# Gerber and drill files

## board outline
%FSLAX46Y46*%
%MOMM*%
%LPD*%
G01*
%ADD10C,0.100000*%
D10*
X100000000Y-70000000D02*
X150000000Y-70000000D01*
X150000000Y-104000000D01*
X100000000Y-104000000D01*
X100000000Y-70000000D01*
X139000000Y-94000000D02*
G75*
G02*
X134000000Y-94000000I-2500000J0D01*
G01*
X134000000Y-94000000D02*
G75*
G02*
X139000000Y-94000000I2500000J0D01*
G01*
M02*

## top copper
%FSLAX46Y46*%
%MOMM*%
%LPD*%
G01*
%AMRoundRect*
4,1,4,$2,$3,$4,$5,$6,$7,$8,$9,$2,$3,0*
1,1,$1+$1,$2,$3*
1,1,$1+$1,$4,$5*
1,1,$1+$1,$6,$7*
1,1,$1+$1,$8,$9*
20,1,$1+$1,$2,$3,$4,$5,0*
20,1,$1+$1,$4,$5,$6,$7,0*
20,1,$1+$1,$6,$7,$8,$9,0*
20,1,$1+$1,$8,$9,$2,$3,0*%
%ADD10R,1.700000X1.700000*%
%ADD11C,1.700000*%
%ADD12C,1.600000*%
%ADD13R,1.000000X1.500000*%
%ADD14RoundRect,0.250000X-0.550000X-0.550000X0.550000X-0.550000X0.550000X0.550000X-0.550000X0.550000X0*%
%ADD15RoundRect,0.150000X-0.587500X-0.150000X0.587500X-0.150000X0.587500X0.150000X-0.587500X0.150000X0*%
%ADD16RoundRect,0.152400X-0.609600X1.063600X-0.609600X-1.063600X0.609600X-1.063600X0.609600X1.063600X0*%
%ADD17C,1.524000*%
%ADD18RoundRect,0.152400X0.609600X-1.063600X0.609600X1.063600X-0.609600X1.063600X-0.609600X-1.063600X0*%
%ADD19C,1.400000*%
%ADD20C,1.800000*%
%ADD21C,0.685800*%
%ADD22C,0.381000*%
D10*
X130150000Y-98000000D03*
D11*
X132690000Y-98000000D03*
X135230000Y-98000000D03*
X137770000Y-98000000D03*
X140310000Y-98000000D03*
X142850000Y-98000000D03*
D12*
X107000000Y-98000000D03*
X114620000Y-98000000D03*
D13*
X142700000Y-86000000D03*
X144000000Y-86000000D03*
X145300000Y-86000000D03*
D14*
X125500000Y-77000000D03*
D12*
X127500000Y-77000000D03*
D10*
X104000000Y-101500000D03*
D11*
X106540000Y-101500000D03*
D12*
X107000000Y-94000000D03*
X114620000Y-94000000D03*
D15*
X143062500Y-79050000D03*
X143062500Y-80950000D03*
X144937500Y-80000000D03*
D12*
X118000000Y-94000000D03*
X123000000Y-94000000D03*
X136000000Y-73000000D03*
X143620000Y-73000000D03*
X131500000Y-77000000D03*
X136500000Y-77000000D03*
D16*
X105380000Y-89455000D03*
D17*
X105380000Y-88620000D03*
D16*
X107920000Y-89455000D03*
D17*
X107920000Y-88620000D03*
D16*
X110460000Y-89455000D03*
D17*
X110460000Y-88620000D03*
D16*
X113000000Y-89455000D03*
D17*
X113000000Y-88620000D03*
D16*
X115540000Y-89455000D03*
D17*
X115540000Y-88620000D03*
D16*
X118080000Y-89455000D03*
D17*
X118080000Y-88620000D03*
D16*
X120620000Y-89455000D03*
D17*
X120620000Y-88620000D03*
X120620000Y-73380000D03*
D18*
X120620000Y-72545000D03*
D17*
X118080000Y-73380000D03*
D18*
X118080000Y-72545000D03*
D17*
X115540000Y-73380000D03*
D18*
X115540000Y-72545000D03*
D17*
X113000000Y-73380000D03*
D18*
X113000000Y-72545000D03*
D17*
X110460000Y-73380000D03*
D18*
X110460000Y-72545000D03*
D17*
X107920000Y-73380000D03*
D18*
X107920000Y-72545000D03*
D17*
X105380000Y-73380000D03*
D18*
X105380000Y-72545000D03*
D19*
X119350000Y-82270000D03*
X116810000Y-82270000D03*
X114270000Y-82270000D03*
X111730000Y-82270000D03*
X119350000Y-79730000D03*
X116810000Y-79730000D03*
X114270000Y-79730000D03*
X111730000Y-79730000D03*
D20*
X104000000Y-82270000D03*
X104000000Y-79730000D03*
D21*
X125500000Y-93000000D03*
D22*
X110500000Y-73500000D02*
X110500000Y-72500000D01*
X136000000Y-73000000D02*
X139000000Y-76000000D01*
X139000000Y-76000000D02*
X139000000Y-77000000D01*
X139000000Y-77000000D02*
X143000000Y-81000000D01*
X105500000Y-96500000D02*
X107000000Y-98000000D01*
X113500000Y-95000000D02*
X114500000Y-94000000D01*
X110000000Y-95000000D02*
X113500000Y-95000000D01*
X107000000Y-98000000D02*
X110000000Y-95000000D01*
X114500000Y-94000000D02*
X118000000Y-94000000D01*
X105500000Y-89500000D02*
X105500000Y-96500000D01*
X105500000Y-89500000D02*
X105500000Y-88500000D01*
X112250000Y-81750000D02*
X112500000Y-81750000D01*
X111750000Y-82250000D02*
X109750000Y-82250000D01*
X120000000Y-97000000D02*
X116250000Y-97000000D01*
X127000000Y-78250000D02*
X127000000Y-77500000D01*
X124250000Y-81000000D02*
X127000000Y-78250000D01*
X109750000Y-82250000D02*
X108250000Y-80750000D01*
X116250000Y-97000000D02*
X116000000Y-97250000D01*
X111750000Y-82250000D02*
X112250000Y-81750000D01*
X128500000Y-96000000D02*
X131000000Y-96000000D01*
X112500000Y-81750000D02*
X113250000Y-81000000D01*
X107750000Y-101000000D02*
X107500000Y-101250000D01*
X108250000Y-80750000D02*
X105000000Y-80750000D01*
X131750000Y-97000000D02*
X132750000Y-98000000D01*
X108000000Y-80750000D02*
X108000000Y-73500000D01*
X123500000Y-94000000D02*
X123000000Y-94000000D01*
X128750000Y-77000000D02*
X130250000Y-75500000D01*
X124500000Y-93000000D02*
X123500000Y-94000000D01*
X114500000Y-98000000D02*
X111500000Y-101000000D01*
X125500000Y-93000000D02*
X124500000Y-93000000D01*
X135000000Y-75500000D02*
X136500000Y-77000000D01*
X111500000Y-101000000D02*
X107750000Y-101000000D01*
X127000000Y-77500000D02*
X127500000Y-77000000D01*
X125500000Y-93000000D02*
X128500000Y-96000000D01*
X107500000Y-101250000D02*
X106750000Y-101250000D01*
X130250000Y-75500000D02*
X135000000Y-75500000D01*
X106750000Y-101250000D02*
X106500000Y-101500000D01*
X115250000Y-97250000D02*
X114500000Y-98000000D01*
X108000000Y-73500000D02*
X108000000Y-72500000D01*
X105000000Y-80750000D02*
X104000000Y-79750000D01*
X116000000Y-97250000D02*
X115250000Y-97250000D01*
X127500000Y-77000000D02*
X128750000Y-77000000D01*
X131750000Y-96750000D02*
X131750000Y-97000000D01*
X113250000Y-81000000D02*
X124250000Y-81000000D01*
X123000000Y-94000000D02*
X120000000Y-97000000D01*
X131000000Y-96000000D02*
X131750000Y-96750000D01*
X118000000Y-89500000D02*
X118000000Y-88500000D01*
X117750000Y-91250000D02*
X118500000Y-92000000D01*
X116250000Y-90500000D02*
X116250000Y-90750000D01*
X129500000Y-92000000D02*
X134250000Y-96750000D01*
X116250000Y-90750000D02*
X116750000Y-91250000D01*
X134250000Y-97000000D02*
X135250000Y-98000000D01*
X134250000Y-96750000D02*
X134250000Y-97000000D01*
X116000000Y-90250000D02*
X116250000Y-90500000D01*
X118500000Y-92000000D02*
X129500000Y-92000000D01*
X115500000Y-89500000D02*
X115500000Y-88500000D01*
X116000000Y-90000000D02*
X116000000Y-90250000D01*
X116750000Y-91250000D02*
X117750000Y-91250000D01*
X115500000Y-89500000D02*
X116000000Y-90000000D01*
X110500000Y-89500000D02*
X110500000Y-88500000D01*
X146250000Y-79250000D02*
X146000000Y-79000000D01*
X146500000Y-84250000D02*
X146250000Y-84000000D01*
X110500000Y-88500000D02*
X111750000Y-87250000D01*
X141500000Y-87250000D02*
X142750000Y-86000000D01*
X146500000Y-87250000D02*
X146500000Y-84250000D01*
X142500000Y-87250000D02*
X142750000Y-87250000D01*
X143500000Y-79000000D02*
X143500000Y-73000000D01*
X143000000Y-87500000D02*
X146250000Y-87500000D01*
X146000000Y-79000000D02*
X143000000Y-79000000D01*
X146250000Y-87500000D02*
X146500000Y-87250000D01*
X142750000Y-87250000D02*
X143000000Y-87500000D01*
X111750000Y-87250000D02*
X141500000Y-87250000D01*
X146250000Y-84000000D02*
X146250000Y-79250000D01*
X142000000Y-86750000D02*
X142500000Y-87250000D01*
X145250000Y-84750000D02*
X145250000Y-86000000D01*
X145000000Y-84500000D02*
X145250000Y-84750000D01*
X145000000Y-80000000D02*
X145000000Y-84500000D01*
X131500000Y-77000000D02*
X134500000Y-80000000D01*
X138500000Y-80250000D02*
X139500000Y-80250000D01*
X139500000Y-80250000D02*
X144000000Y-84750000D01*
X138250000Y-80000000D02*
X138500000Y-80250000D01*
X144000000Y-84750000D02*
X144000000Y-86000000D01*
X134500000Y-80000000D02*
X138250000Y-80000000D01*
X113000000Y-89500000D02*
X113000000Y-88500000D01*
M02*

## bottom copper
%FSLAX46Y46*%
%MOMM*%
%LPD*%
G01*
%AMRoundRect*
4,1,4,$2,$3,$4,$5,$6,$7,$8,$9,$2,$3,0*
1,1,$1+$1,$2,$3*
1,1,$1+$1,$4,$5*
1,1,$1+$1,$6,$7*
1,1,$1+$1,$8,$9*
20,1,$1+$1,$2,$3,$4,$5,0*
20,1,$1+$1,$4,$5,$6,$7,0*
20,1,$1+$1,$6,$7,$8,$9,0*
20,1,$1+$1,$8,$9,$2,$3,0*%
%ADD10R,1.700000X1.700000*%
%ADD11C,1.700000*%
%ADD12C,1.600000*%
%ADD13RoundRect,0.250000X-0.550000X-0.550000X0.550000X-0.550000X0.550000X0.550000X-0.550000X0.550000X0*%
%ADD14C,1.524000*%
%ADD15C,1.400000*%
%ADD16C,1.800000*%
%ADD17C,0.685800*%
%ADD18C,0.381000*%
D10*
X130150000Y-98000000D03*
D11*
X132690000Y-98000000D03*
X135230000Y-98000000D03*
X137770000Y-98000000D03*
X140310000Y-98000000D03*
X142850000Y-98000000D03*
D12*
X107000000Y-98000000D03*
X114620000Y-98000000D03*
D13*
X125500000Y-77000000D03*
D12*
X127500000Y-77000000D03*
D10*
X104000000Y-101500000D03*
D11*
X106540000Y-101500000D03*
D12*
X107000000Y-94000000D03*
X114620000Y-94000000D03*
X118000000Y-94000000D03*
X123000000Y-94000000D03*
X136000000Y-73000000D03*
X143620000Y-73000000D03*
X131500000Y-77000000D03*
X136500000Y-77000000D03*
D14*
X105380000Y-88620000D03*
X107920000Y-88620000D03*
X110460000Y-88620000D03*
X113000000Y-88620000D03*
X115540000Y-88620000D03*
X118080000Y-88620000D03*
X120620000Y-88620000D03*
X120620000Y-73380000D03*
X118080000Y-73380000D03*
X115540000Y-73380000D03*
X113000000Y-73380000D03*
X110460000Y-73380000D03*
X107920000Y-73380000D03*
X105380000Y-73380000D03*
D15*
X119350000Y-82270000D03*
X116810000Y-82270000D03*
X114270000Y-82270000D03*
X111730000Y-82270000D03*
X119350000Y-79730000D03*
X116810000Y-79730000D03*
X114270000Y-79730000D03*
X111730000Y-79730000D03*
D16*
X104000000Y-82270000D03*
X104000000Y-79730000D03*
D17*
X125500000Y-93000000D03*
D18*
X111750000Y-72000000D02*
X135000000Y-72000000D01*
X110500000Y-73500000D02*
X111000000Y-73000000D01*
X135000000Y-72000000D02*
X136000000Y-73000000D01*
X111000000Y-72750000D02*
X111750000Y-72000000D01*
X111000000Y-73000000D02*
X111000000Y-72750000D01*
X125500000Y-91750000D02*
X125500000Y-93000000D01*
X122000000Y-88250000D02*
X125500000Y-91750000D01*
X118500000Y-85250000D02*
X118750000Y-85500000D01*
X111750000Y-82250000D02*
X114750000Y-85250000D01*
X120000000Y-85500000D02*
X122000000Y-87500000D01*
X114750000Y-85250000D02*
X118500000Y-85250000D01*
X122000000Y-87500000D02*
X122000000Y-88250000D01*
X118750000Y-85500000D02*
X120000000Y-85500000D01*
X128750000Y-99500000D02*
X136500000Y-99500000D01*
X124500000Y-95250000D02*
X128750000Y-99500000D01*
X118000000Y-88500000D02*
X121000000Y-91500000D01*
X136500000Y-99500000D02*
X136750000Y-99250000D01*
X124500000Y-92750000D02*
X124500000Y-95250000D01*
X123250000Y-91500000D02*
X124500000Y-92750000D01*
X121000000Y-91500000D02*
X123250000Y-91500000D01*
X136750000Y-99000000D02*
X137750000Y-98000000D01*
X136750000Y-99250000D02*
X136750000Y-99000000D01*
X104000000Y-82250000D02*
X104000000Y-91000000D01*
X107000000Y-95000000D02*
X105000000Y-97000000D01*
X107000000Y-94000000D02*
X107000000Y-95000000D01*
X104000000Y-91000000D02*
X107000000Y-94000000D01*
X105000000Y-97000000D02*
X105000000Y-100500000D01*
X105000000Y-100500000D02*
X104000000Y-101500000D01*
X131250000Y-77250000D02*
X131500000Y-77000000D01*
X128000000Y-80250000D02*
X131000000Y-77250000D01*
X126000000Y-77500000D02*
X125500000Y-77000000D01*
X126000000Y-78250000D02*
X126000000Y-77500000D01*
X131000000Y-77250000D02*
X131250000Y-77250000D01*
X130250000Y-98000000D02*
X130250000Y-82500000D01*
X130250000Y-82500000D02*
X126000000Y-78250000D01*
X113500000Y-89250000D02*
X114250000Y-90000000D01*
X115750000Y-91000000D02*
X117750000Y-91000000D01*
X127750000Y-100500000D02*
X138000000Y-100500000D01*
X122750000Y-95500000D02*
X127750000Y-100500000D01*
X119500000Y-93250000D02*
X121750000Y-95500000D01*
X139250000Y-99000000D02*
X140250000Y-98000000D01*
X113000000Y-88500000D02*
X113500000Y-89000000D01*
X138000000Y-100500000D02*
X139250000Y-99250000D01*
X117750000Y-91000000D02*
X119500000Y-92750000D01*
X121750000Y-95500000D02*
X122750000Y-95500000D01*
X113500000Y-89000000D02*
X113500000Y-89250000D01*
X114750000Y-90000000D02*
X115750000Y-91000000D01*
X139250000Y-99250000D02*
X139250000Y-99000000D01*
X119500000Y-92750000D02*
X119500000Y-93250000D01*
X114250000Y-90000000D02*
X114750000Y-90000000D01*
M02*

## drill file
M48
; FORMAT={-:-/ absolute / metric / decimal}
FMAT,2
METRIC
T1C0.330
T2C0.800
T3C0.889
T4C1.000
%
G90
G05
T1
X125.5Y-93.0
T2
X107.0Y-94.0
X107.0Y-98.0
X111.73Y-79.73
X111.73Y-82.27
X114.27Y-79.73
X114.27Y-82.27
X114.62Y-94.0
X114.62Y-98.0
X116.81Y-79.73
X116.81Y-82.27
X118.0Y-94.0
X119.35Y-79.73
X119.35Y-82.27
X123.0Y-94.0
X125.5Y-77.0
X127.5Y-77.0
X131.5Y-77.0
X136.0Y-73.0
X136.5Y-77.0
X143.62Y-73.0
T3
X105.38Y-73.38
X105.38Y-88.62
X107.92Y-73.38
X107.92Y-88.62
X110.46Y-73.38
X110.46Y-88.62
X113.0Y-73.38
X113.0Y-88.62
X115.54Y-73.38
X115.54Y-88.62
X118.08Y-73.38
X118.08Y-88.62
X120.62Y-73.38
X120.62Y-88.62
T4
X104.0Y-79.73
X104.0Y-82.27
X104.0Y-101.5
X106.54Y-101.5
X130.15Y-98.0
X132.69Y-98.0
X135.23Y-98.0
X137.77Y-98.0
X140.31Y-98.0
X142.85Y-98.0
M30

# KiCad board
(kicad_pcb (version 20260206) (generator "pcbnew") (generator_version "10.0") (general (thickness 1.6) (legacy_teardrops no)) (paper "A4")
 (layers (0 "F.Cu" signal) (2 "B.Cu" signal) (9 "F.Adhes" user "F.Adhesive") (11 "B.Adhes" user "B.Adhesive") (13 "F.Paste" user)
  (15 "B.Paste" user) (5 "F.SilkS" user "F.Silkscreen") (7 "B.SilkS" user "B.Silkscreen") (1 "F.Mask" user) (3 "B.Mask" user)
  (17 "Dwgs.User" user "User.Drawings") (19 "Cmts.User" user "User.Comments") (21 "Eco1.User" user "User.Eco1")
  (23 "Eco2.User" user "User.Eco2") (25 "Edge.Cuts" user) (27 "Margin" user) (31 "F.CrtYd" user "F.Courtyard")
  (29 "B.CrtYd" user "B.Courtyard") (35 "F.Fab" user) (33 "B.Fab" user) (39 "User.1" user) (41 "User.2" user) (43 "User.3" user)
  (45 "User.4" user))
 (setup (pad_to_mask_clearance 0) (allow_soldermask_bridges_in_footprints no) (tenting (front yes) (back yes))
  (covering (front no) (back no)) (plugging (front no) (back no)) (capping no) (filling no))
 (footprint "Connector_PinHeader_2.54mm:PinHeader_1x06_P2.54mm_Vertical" (layer "F.Cu") (at 130.15 98 90)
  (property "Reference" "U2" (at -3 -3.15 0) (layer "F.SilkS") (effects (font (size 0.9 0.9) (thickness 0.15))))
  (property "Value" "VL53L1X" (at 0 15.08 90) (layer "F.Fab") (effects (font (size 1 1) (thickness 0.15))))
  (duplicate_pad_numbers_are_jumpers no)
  (pad "1" thru_hole rect (at 0 0 90) (size 1.7 1.7) (drill 1) (layers "*.Cu" "*.Mask") (remove_unused_layers no) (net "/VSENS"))
  (pad "2" thru_hole circle (at 0 2.54 90) (size 1.7 1.7) (drill 1) (layers "*.Cu" "*.Mask") (remove_unused_layers no) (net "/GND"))
  (pad "3" thru_hole circle (at 0 5.08 90) (size 1.7 1.7) (drill 1) (layers "*.Cu" "*.Mask") (remove_unused_layers no) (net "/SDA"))
  (pad "4" thru_hole circle (at 0 7.62 90) (size 1.7 1.7) (drill 1) (layers "*.Cu" "*.Mask") (remove_unused_layers no) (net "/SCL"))
  (pad "5" thru_hole circle (at 0 10.16 90) (size 1.7 1.7) (drill 1) (layers "*.Cu" "*.Mask") (remove_unused_layers no) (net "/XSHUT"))
  (pad "6" thru_hole circle (at 0 12.7 90) (size 1.7 1.7) (drill 1) (layers "*.Cu" "*.Mask") (remove_unused_layers no)
   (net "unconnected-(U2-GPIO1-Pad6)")))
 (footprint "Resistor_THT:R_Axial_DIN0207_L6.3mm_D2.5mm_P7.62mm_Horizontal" (layer "F.Cu") (at 107 98)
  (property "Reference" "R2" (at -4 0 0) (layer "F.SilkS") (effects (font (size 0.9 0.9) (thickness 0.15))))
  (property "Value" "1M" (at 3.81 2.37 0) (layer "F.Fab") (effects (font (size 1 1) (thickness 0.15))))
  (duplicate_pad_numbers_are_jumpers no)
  (pad "1" thru_hole circle (at 0 0) (size 1.6 1.6) (drill 0.8) (layers "*.Cu" "*.Mask") (remove_unused_layers no) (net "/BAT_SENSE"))
  (pad "2" thru_hole circle (at 7.62 0) (size 1.6 1.6) (drill 0.8) (layers "*.Cu" "*.Mask") (remove_unused_layers no) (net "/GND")))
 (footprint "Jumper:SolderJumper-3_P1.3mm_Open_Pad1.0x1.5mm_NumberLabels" (layer "F.Cu") (at 144 86)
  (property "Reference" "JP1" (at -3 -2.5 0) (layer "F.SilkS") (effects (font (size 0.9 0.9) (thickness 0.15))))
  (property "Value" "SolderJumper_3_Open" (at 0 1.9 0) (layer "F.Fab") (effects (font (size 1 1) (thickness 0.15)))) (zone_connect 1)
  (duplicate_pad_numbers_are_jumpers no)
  (pad "1" smd rect (at -1.3 0) (size 1 1.5) (layers "F.Cu" "F.Mask") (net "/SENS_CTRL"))
  (pad "2" smd rect (at 0 0) (size 1 1.5) (layers "F.Cu" "F.Mask") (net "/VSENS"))
  (pad "3" smd rect (at 1.3 0) (size 1 1.5) (layers "F.Cu" "F.Mask") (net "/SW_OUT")))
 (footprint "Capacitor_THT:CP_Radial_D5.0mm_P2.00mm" (layer "F.Cu") (at 125.5 77)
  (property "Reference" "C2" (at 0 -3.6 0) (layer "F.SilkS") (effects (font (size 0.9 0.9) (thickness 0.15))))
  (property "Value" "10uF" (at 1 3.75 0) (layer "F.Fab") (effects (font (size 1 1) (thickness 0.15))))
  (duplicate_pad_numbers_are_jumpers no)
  (pad "1" thru_hole roundrect (at 0 0) (size 1.6 1.6) (drill 0.8) (layers "*.Cu" "*.Mask") (remove_unused_layers no)
   (roundrect_rratio 0.15625) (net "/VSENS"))
  (pad "2" thru_hole circle (at 2 0) (size 1.6 1.6) (drill 0.8) (layers "*.Cu" "*.Mask") (remove_unused_layers no) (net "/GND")))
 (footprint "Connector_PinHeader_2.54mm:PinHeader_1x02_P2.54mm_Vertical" (layer "F.Cu") (at 104 101.5 90)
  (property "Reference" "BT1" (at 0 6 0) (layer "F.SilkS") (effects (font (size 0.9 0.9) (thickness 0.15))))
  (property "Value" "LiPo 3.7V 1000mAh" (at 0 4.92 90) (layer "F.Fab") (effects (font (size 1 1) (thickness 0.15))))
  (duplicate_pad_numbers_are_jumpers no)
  (pad "1" thru_hole rect (at 0 0 90) (size 1.7 1.7) (drill 1) (layers "*.Cu" "*.Mask") (remove_unused_layers no) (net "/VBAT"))
  (pad "2" thru_hole circle (at 0 2.54 90) (size 1.7 1.7) (drill 1) (layers "*.Cu" "*.Mask") (remove_unused_layers no) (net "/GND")))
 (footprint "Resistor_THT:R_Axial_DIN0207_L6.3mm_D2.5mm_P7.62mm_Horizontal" (layer "F.Cu") (at 107 94)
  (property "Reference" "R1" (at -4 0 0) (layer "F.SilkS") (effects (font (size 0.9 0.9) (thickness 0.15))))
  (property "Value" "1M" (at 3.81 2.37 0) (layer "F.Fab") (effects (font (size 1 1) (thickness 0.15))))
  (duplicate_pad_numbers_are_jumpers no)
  (pad "1" thru_hole circle (at 0 0) (size 1.6 1.6) (drill 0.8) (layers "*.Cu" "*.Mask") (remove_unused_layers no) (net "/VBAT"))
  (pad "2" thru_hole circle (at 7.62 0) (size 1.6 1.6) (drill 0.8) (layers "*.Cu" "*.Mask") (remove_unused_layers no) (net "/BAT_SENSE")))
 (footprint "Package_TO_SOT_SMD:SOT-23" (layer "F.Cu") (at 144 80)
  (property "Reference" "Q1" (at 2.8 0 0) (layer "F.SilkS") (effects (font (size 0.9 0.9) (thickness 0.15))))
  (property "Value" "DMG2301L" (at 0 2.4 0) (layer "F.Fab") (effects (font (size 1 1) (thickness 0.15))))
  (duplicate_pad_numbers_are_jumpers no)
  (pad "1" smd roundrect (at -0.9375 -0.95) (size 1.475 0.6) (layers "F.Cu" "F.Mask" "F.Paste") (roundrect_rratio 0.25) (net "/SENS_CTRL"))
  (pad "2" smd roundrect (at -0.9375 0.95) (size 1.475 0.6) (layers "F.Cu" "F.Mask" "F.Paste") (roundrect_rratio 0.25) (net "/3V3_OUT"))
  (pad "3" smd roundrect (at 0.9375 0) (size 1.475 0.6) (layers "F.Cu" "F.Mask" "F.Paste") (roundrect_rratio 0.25) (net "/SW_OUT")))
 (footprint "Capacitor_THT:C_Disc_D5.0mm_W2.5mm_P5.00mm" (layer "F.Cu") (at 118 94)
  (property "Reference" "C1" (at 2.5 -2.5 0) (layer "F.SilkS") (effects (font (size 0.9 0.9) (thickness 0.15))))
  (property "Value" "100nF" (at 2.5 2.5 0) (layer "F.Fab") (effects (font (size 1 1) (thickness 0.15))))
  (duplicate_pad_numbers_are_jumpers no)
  (pad "1" thru_hole circle (at 0 0) (size 1.6 1.6) (drill 0.8) (layers "*.Cu" "*.Mask") (remove_unused_layers no) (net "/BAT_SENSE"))
  (pad "2" thru_hole circle (at 5 0) (size 1.6 1.6) (drill 0.8) (layers "*.Cu" "*.Mask") (remove_unused_layers no) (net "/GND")))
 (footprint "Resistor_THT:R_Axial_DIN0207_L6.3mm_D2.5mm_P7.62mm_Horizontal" (layer "F.Cu") (at 136 73)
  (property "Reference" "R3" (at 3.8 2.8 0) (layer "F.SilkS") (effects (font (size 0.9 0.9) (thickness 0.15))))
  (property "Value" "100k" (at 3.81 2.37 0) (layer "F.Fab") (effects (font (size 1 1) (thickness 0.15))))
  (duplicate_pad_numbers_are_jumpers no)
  (pad "1" thru_hole circle (at 0 0) (size 1.6 1.6) (drill 0.8) (layers "*.Cu" "*.Mask") (remove_unused_layers no) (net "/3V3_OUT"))
  (pad "2" thru_hole circle (at 7.62 0) (size 1.6 1.6) (drill 0.8) (layers "*.Cu" "*.Mask") (remove_unused_layers no) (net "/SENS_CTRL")))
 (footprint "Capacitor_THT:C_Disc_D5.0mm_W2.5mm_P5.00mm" (layer "F.Cu") (at 131.5 77)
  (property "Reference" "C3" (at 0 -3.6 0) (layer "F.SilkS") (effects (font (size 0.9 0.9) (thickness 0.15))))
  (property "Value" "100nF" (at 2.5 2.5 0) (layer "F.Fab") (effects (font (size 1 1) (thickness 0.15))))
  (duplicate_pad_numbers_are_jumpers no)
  (pad "1" thru_hole circle (at 0 0) (size 1.6 1.6) (drill 0.8) (layers "*.Cu" "*.Mask") (remove_unused_layers no) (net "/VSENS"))
  (pad "2" thru_hole circle (at 5 0) (size 1.6 1.6) (drill 0.8) (layers "*.Cu" "*.Mask") (remove_unused_layers no) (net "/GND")))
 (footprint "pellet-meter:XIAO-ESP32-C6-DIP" (layer "F.Cu") (at 113 81 180)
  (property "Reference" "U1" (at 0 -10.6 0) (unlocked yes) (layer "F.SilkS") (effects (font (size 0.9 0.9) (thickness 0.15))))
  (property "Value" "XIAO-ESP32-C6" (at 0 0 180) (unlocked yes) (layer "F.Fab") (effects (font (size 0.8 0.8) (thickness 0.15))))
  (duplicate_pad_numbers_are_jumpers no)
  (pad "1" smd roundrect (at 7.62 -8.455 270) (size 2.432 1.524) (layers "F.Cu" "F.Mask") (roundrect_rratio 0.1) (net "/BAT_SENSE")
   (thermal_bridge_angle 45))
  (pad "1" thru_hole circle (at 7.62 -7.62 270) (size 1.524 1.524) (drill 0.889) (layers "*.Cu" "*.Mask") (remove_unused_layers no)
   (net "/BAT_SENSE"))
  (pad "2" smd roundrect (at 5.08 -8.455 270) (size 2.432 1.524) (layers "F.Cu" "F.Mask") (roundrect_rratio 0.1)
   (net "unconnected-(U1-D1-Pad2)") (thermal_bridge_angle 45))
  (pad "2" thru_hole circle (at 5.08 -7.62 270) (size 1.524 1.524) (drill 0.889) (layers "*.Cu" "*.Mask") (remove_unused_layers no)
   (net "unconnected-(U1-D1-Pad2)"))
  (pad "3" smd roundrect (at 2.54 -8.455 270) (size 2.432 1.524) (layers "F.Cu" "F.Mask") (roundrect_rratio 0.1) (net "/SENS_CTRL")
   (thermal_bridge_angle 45))
  (pad "3" thru_hole circle (at 2.54 -7.62 270) (size 1.524 1.524) (drill 0.889) (layers "*.Cu" "*.Mask") (remove_unused_layers no)
   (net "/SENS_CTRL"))
  (pad "4" smd roundrect (at 0 -8.455 270) (size 2.432 1.524) (layers "F.Cu" "F.Mask") (roundrect_rratio 0.1) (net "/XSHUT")
   (thermal_bridge_angle 45))
  (pad "4" thru_hole circle (at 0 -7.62 270) (size 1.524 1.524) (drill 0.889) (layers "*.Cu" "*.Mask") (remove_unused_layers no)
   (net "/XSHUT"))
  (pad "5" smd roundrect (at -2.54 -8.455 270) (size 2.432 1.524) (layers "F.Cu" "F.Mask") (roundrect_rratio 0.1) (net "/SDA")
   (thermal_bridge_angle 45))
  (pad "5" thru_hole circle (at -2.54 -7.62 270) (size 1.524 1.524) (drill 0.889) (layers "*.Cu" "*.Mask") (remove_unused_layers no)
   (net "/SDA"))
  (pad "6" smd roundrect (at -5.08 -8.455 270) (size 2.432 1.524) (layers "F.Cu" "F.Mask") (roundrect_rratio 0.1) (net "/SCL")
   (thermal_bridge_angle 45))
  (pad "6" thru_hole circle (at -5.08 -7.62 270) (size 1.524 1.524) (drill 0.889) (layers "*.Cu" "*.Mask") (remove_unused_layers no)
   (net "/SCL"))
  (pad "7" smd roundrect (at -7.62 -8.455 270) (size 2.432 1.524) (layers "F.Cu" "F.Mask") (roundrect_rratio 0.1)
   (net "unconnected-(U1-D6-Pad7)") (thermal_bridge_angle 45))
  (pad "7" thru_hole circle (at -7.62 -7.62 270) (size 1.524 1.524) (drill 0.889) (layers "*.Cu" "*.Mask") (remove_unused_layers no)
   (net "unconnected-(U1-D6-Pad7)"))
  (pad "8" thru_hole circle (at -7.62 7.62 90) (size 1.524 1.524) (drill 0.889) (layers "*.Cu" "*.Mask") (remove_unused_layers no)
   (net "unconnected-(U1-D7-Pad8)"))
  (pad "8" smd roundrect (at -7.62 8.455 90) (size 2.432 1.524) (layers "F.Cu" "F.Mask") (roundrect_rratio 0.1)
   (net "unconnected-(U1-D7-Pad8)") (thermal_bridge_angle 45))
  (pad "9" thru_hole circle (at -5.08 7.62 90) (size 1.524 1.524) (drill 0.889) (layers "*.Cu" "*.Mask") (remove_unused_layers no)
   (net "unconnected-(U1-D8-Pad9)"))
  (pad "9" smd roundrect (at -5.08 8.455 90) (size 2.432 1.524) (layers "F.Cu" "F.Mask") (roundrect_rratio 0.1)
   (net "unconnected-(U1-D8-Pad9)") (thermal_bridge_angle 45))
  (pad "10" thru_hole circle (at -2.54 7.62 90) (size 1.524 1.524) (drill 0.889) (layers "*.Cu" "*.Mask") (remove_unused_layers no)
   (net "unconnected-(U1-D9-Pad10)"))
  (pad "10" smd roundrect (at -2.54 8.455 90) (size 2.432 1.524) (layers "F.Cu" "F.Mask") (roundrect_rratio 0.1)
   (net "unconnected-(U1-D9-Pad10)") (thermal_bridge_angle 45))
  (pad "11" thru_hole circle (at 0 7.62 90) (size 1.524 1.524) (drill 0.889) (layers "*.Cu" "*.Mask") (remove_unused_layers no)
   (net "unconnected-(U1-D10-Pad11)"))
  (pad "11" smd roundrect (at 0 8.455 90) (size 2.432 1.524) (layers "F.Cu" "F.Mask") (roundrect_rratio 0.1)
   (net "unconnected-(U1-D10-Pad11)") (thermal_bridge_angle 45))
  (pad "12" thru_hole circle (at 2.54 7.62 90) (size 1.524 1.524) (drill 0.889) (layers "*.Cu" "*.Mask") (remove_unused_layers no)
   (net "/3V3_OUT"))
  (pad "12" smd roundrect (at 2.54 8.455 90) (size 2.432 1.524) (layers "F.Cu" "F.Mask") (roundrect_rratio 0.1) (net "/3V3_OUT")
   (thermal_bridge_angle 45))
  (pad "13" thru_hole circle (at 5.08 7.62 90) (size 1.524 1.524) (drill 0.889) (layers "*.Cu" "*.Mask") (remove_unused_layers no)
   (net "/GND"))
  (pad "13" smd roundrect (at 5.08 8.455 90) (size 2.432 1.524) (layers "F.Cu" "F.Mask") (roundrect_rratio 0.1) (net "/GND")
   (thermal_bridge_angle 45))
  (pad "14" thru_hole circle (at 7.62 7.62 90) (size 1.524 1.524) (drill 0.889) (layers "*.Cu" "*.Mask") (remove_unused_layers no)
   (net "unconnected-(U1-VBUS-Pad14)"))
  (pad "14" smd roundrect (at 7.62 8.455 90) (size 2.432 1.524) (layers "F.Cu" "F.Mask") (roundrect_rratio 0.1)
   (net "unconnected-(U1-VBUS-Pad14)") (thermal_bridge_angle 45))
  (pad "15" thru_hole circle (at -6.35 -1.27 270) (size 1.4 1.4) (drill 0.8) (layers "*.Cu" "*.Mask") (remove_unused_layers no)
   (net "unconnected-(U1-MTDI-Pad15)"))
  (pad "16" thru_hole circle (at -3.81 -1.27 270) (size 1.4 1.4) (drill 0.8) (layers "*.Cu" "*.Mask") (remove_unused_layers no)
   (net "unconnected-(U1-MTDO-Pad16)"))
  (pad "17" thru_hole circle (at -1.27 -1.27 270) (size 1.4 1.4) (drill 0.8) (layers "*.Cu" "*.Mask") (remove_unused_layers no)
   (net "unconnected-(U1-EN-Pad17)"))
  (pad "18" thru_hole circle (at 1.27 -1.27 270) (size 1.4 1.4) (drill 0.8) (layers "*.Cu" "*.Mask") (remove_unused_layers no) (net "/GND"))
  (pad "19" thru_hole circle (at -6.35 1.27 270) (size 1.4 1.4) (drill 0.8) (layers "*.Cu" "*.Mask") (remove_unused_layers no)
   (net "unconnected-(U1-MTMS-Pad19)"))
  (pad "20" thru_hole circle (at -3.81 1.27 270) (size 1.4 1.4) (drill 0.8) (layers "*.Cu" "*.Mask") (remove_unused_layers no)
   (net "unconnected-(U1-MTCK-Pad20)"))
  (pad "21" thru_hole circle (at -1.27 1.27 270) (size 1.4 1.4) (drill 0.8) (layers "*.Cu" "*.Mask") (remove_unused_layers no)
   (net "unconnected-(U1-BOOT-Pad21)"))
  (pad "22" thru_hole circle (at 1.27 1.27 270) (size 1.4 1.4) (drill 0.8) (layers "*.Cu" "*.Mask") (remove_unused_layers no)
   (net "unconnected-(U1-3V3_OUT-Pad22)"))
  (pad "23" thru_hole circle (at 9 -1.27 270) (size 1.8 1.8) (drill 1) (layers "*.Cu" "*.Mask") (remove_unused_layers no) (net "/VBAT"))
  (pad "24" thru_hole circle (at 9 1.27 270) (size 1.8 1.8) (drill 1) (layers "*.Cu" "*.Mask") (remove_unused_layers no) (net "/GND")))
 (gr_rect (start 100 70) (end 150 104) (stroke (width 0.1) (type default)) (fill no) (layer "Edge.Cuts"))
 (gr_circle (center 136.5 94) (end 139 94) (stroke (width 0.1) (type default)) (fill no) (layer "Edge.Cuts"))
 (segment (start 110.5 73.5) (end 110.5 72.5) (width 0.381) (layer "F.Cu") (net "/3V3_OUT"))
 (segment (start 136 73) (end 139 76) (width 0.381) (layer "F.Cu") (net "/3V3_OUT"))
 (segment (start 139 76) (end 139 77) (width 0.381) (layer "F.Cu") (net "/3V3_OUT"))
 (segment (start 139 77) (end 143 81) (width 0.381) (layer "F.Cu") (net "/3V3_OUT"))
 (segment (start 111.75 72) (end 135 72) (width 0.381) (layer "B.Cu") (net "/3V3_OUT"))
 (segment (start 110.5 73.5) (end 111 73) (width 0.381) (layer "B.Cu") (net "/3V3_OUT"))
 (segment (start 135 72) (end 136 73) (width 0.381) (layer "B.Cu") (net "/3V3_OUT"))
 (segment (start 111 72.75) (end 111.75 72) (width 0.381) (layer "B.Cu") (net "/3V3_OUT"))
 (segment (start 111 73) (end 111 72.75) (width 0.381) (layer "B.Cu") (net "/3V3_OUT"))
 (segment (start 105.5 96.5) (end 107 98) (width 0.381) (layer "F.Cu") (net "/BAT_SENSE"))
 (segment (start 113.5 95) (end 114.5 94) (width 0.381) (layer "F.Cu") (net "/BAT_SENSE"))
 (segment (start 110 95) (end 113.5 95) (width 0.381) (layer "F.Cu") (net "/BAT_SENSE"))
 (segment (start 107 98) (end 110 95) (width 0.381) (layer "F.Cu") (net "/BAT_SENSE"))
 (segment (start 114.5 94) (end 118 94) (width 0.381) (layer "F.Cu") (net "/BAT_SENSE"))
 (segment (start 105.5 89.5) (end 105.5 96.5) (width 0.381) (layer "F.Cu") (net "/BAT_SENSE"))
 (segment (start 105.5 89.5) (end 105.5 88.5) (width 0.381) (layer "F.Cu") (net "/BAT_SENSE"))
 (segment (start 112.25 81.75) (end 112.5 81.75) (width 0.381) (layer "F.Cu") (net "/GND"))
 (segment (start 111.75 82.25) (end 109.75 82.25) (width 0.381) (layer "F.Cu") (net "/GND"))
 (segment (start 120 97) (end 116.25 97) (width 0.381) (layer "F.Cu") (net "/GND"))
 (segment (start 127 78.25) (end 127 77.5) (width 0.381) (layer "F.Cu") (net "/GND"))
 (segment (start 124.25 81) (end 127 78.25) (width 0.381) (layer "F.Cu") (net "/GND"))
 (segment (start 109.75 82.25) (end 108.25 80.75) (width 0.381) (layer "F.Cu") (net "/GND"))
 (segment (start 116.25 97) (end 116 97.25) (width 0.381) (layer "F.Cu") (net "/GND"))
 (segment (start 111.75 82.25) (end 112.25 81.75) (width 0.381) (layer "F.Cu") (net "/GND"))
 (segment (start 128.5 96) (end 131 96) (width 0.381) (layer "F.Cu") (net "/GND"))
 (segment (start 112.5 81.75) (end 113.25 81) (width 0.381) (layer "F.Cu") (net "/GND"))
 (segment (start 107.75 101) (end 107.5 101.25) (width 0.381) (layer "F.Cu") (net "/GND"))
 (segment (start 108.25 80.75) (end 105 80.75) (width 0.381) (layer "F.Cu") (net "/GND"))
 (segment (start 131.75 97) (end 132.75 98) (width 0.381) (layer "F.Cu") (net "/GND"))
 (segment (start 108 80.75) (end 108 73.5) (width 0.381) (layer "F.Cu") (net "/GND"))
 (segment (start 123.5 94) (end 123 94) (width 0.381) (layer "F.Cu") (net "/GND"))
 (segment (start 128.75 77) (end 130.25 75.5) (width 0.381) (layer "F.Cu") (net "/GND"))
 (segment (start 124.5 93) (end 123.5 94) (width 0.381) (layer "F.Cu") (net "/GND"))
 (segment (start 114.5 98) (end 111.5 101) (width 0.381) (layer "F.Cu") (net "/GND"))
 (segment (start 125.5 93) (end 124.5 93) (width 0.381) (layer "F.Cu") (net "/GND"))
 (segment (start 135 75.5) (end 136.5 77) (width 0.381) (layer "F.Cu") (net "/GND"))
 (segment (start 111.5 101) (end 107.75 101) (width 0.381) (layer "F.Cu") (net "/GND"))
 (segment (start 127 77.5) (end 127.5 77) (width 0.381) (layer "F.Cu") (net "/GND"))
 (segment (start 125.5 93) (end 128.5 96) (width 0.381) (layer "F.Cu") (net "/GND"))
 (segment (start 107.5 101.25) (end 106.75 101.25) (width 0.381) (layer "F.Cu") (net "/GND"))
 (segment (start 130.25 75.5) (end 135 75.5) (width 0.381) (layer "F.Cu") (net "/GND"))
 (segment (start 106.75 101.25) (end 106.5 101.5) (width 0.381) (layer "F.Cu") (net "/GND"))
 (segment (start 115.25 97.25) (end 114.5 98) (width 0.381) (layer "F.Cu") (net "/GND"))
 (segment (start 108 73.5) (end 108 72.5) (width 0.381) (layer "F.Cu") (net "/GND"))
 (segment (start 105 80.75) (end 104 79.75) (width 0.381) (layer "F.Cu") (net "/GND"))
 (segment (start 116 97.25) (end 115.25 97.25) (width 0.381) (layer "F.Cu") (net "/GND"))
 (segment (start 127.5 77) (end 128.75 77) (width 0.381) (layer "F.Cu") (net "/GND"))
 (segment (start 131.75 96.75) (end 131.75 97) (width 0.381) (layer "F.Cu") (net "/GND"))
 (segment (start 113.25 81) (end 124.25 81) (width 0.381) (layer "F.Cu") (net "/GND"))
 (segment (start 123 94) (end 120 97) (width 0.381) (layer "F.Cu") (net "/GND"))
 (segment (start 131 96) (end 131.75 96.75) (width 0.381) (layer "F.Cu") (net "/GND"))
 (via (at 125.5 93) (size 0.6858) (drill 0.3302) (layers "F.Cu" "B.Cu") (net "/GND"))
 (segment (start 125.5 91.75) (end 125.5 93) (width 0.381) (layer "B.Cu") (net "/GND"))
 (segment (start 122 88.25) (end 125.5 91.75) (width 0.381) (layer "B.Cu") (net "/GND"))
 (segment (start 118.5 85.25) (end 118.75 85.5) (width 0.381) (layer "B.Cu") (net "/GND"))
 (segment (start 111.75 82.25) (end 114.75 85.25) (width 0.381) (layer "B.Cu") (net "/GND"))
 (segment (start 120 85.5) (end 122 87.5) (width 0.381) (layer "B.Cu") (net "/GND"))
 (segment (start 114.75 85.25) (end 118.5 85.25) (width 0.381) (layer "B.Cu") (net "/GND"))
 (segment (start 122 87.5) (end 122 88.25) (width 0.381) (layer "B.Cu") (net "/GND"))
 (segment (start 118.75 85.5) (end 120 85.5) (width 0.381) (layer "B.Cu") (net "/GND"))
 (segment (start 118 89.5) (end 118 88.5) (width 0.381) (layer "F.Cu") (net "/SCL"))
 (segment (start 128.75 99.5) (end 136.5 99.5) (width 0.381) (layer "B.Cu") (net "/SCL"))
 (segment (start 124.5 95.25) (end 128.75 99.5) (width 0.381) (layer "B.Cu") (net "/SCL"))
 (segment (start 118 88.5) (end 121 91.5) (width 0.381) (layer "B.Cu") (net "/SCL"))
 (segment (start 136.5 99.5) (end 136.75 99.25) (width 0.381) (layer "B.Cu") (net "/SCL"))
 (segment (start 124.5 92.75) (end 124.5 95.25) (width 0.381) (layer "B.Cu") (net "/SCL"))
 (segment (start 123.25 91.5) (end 124.5 92.75) (width 0.381) (layer "B.Cu") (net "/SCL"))
 (segment (start 121 91.5) (end 123.25 91.5) (width 0.381) (layer "B.Cu") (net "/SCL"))
 (segment (start 136.75 99) (end 137.75 98) (width 0.381) (layer "B.Cu") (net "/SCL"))
 (segment (start 136.75 99.25) (end 136.75 99) (width 0.381) (layer "B.Cu") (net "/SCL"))
 (segment (start 117.75 91.25) (end 118.5 92) (width 0.381) (layer "F.Cu") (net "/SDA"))
 (segment (start 116.25 90.5) (end 116.25 90.75) (width 0.381) (layer "F.Cu") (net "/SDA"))
 (segment (start 129.5 92) (end 134.25 96.75) (width 0.381) (layer "F.Cu") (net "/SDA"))
 (segment (start 116.25 90.75) (end 116.75 91.25) (width 0.381) (layer "F.Cu") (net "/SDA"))
 (segment (start 134.25 97) (end 135.25 98) (width 0.381) (layer "F.Cu") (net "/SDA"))
 (segment (start 134.25 96.75) (end 134.25 97) (width 0.381) (layer "F.Cu") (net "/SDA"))
 (segment (start 116 90.25) (end 116.25 90.5) (width 0.381) (layer "F.Cu") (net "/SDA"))
 (segment (start 118.5 92) (end 129.5 92) (width 0.381) (layer "F.Cu") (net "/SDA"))
 (segment (start 115.5 89.5) (end 115.5 88.5) (width 0.381) (layer "F.Cu") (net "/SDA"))
 (segment (start 116 90) (end 116 90.25) (width 0.381) (layer "F.Cu") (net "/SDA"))
 (segment (start 116.75 91.25) (end 117.75 91.25) (width 0.381) (layer "F.Cu") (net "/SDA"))
 (segment (start 115.5 89.5) (end 116 90) (width 0.381) (layer "F.Cu") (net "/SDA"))
 (segment (start 110.5 89.5) (end 110.5 88.5) (width 0.381) (layer "F.Cu") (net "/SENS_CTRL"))
 (segment (start 146.25 79.25) (end 146 79) (width 0.381) (layer "F.Cu") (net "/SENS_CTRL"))
 (segment (start 146.5 84.25) (end 146.25 84) (width 0.381) (layer "F.Cu") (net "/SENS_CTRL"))
 (segment (start 110.5 88.5) (end 111.75 87.25) (width 0.381) (layer "F.Cu") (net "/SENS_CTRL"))
 (segment (start 141.5 87.25) (end 142.75 86) (width 0.381) (layer "F.Cu") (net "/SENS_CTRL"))
 (segment (start 146.5 87.25) (end 146.5 84.25) (width 0.381) (layer "F.Cu") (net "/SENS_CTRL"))
 (segment (start 142.5 87.25) (end 142.75 87.25) (width 0.381) (layer "F.Cu") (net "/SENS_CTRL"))
 (segment (start 143.5 79) (end 143.5 73) (width 0.381) (layer "F.Cu") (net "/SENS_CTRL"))
 (segment (start 143 87.5) (end 146.25 87.5) (width 0.381) (layer "F.Cu") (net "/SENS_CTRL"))
 (segment (start 146 79) (end 143 79) (width 0.381) (layer "F.Cu") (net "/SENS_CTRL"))
 (segment (start 146.25 87.5) (end 146.5 87.25) (width 0.381) (layer "F.Cu") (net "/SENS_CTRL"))
 (segment (start 142.75 87.25) (end 143 87.5) (width 0.381) (layer "F.Cu") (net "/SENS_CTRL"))
 (segment (start 111.75 87.25) (end 141.5 87.25) (width 0.381) (layer "F.Cu") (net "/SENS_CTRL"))
 (segment (start 146.25 84) (end 146.25 79.25) (width 0.381) (layer "F.Cu") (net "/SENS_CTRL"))
 (segment (start 142 86.75) (end 142.5 87.25) (width 0.381) (layer "F.Cu") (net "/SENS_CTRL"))
 (segment (start 145.25 84.75) (end 145.25 86) (width 0.381) (layer "F.Cu") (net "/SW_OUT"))
 (segment (start 145 84.5) (end 145.25 84.75) (width 0.381) (layer "F.Cu") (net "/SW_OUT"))
 (segment (start 145 80) (end 145 84.5) (width 0.381) (layer "F.Cu") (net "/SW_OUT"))
 (segment (start 104 82.25) (end 104 91) (width 0.381) (layer "B.Cu") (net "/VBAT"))
 (segment (start 107 95) (end 105 97) (width 0.381) (layer "B.Cu") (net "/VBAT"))
 (segment (start 107 94) (end 107 95) (width 0.381) (layer "B.Cu") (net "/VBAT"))
 (segment (start 104 91) (end 107 94) (width 0.381) (layer "B.Cu") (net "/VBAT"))
 (segment (start 105 97) (end 105 100.5) (width 0.381) (layer "B.Cu") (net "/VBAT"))
 (segment (start 105 100.5) (end 104 101.5) (width 0.381) (layer "B.Cu") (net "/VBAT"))
 (segment (start 131.5 77) (end 134.5 80) (width 0.381) (layer "F.Cu") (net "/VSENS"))
 (segment (start 138.5 80.25) (end 139.5 80.25) (width 0.381) (layer "F.Cu") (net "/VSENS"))
 (segment (start 139.5 80.25) (end 144 84.75) (width 0.381) (layer "F.Cu") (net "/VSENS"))
 (segment (start 138.25 80) (end 138.5 80.25) (width 0.381) (layer "F.Cu") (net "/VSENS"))
 (segment (start 144 84.75) (end 144 86) (width 0.381) (layer "F.Cu") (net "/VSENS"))
 (segment (start 134.5 80) (end 138.25 80) (width 0.381) (layer "F.Cu") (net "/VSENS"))
 (segment (start 131.25 77.25) (end 131.5 77) (width 0.381) (layer "B.Cu") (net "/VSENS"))
 (segment (start 128 80.25) (end 131 77.25) (width 0.381) (layer "B.Cu") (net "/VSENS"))
 (segment (start 126 77.5) (end 125.5 77) (width 0.381) (layer "B.Cu") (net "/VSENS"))
 (segment (start 126 78.25) (end 126 77.5) (width 0.381) (layer "B.Cu") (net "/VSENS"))
 (segment (start 131 77.25) (end 131.25 77.25) (width 0.381) (layer "B.Cu") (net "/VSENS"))
 (segment (start 130.25 98) (end 130.25 82.5) (width 0.381) (layer "B.Cu") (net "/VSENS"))
 (segment (start 130.25 82.5) (end 126 78.25) (width 0.381) (layer "B.Cu") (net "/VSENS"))
 (segment (start 113 89.5) (end 113 88.5) (width 0.381) (layer "F.Cu") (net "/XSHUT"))
 (segment (start 113.5 89.25) (end 114.25 90) (width 0.381) (layer "B.Cu") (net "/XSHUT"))
 (segment (start 115.75 91) (end 117.75 91) (width 0.381) (layer "B.Cu") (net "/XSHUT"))
 (segment (start 127.75 100.5) (end 138 100.5) (width 0.381) (layer "B.Cu") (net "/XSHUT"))
 (segment (start 122.75 95.5) (end 127.75 100.5) (width 0.381) (layer "B.Cu") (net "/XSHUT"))
 (segment (start 119.5 93.25) (end 121.75 95.5) (width 0.381) (layer "B.Cu") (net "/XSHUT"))
 (segment (start 139.25 99) (end 140.25 98) (width 0.381) (layer "B.Cu") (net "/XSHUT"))
 (segment (start 113 88.5) (end 113.5 89) (width 0.381) (layer "B.Cu") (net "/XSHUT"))
 (segment (start 138 100.5) (end 139.25 99.25) (width 0.381) (layer "B.Cu") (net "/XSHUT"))
 (segment (start 117.75 91) (end 119.5 92.75) (width 0.381) (layer "B.Cu") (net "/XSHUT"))
 (segment (start 121.75 95.5) (end 122.75 95.5) (width 0.381) (layer "B.Cu") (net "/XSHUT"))
 (segment (start 113.5 89) (end 113.5 89.25) (width 0.381) (layer "B.Cu") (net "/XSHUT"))
 (segment (start 114.75 90) (end 115.75 91) (width 0.381) (layer "B.Cu") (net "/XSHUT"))
 (segment (start 139.25 99.25) (end 139.25 99) (width 0.381) (layer "B.Cu") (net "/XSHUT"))
 (segment (start 119.5 92.75) (end 119.5 93.25) (width 0.381) (layer "B.Cu") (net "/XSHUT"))
 (segment (start 114.25 90) (end 114.75 90) (width 0.381) (layer "B.Cu") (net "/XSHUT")))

